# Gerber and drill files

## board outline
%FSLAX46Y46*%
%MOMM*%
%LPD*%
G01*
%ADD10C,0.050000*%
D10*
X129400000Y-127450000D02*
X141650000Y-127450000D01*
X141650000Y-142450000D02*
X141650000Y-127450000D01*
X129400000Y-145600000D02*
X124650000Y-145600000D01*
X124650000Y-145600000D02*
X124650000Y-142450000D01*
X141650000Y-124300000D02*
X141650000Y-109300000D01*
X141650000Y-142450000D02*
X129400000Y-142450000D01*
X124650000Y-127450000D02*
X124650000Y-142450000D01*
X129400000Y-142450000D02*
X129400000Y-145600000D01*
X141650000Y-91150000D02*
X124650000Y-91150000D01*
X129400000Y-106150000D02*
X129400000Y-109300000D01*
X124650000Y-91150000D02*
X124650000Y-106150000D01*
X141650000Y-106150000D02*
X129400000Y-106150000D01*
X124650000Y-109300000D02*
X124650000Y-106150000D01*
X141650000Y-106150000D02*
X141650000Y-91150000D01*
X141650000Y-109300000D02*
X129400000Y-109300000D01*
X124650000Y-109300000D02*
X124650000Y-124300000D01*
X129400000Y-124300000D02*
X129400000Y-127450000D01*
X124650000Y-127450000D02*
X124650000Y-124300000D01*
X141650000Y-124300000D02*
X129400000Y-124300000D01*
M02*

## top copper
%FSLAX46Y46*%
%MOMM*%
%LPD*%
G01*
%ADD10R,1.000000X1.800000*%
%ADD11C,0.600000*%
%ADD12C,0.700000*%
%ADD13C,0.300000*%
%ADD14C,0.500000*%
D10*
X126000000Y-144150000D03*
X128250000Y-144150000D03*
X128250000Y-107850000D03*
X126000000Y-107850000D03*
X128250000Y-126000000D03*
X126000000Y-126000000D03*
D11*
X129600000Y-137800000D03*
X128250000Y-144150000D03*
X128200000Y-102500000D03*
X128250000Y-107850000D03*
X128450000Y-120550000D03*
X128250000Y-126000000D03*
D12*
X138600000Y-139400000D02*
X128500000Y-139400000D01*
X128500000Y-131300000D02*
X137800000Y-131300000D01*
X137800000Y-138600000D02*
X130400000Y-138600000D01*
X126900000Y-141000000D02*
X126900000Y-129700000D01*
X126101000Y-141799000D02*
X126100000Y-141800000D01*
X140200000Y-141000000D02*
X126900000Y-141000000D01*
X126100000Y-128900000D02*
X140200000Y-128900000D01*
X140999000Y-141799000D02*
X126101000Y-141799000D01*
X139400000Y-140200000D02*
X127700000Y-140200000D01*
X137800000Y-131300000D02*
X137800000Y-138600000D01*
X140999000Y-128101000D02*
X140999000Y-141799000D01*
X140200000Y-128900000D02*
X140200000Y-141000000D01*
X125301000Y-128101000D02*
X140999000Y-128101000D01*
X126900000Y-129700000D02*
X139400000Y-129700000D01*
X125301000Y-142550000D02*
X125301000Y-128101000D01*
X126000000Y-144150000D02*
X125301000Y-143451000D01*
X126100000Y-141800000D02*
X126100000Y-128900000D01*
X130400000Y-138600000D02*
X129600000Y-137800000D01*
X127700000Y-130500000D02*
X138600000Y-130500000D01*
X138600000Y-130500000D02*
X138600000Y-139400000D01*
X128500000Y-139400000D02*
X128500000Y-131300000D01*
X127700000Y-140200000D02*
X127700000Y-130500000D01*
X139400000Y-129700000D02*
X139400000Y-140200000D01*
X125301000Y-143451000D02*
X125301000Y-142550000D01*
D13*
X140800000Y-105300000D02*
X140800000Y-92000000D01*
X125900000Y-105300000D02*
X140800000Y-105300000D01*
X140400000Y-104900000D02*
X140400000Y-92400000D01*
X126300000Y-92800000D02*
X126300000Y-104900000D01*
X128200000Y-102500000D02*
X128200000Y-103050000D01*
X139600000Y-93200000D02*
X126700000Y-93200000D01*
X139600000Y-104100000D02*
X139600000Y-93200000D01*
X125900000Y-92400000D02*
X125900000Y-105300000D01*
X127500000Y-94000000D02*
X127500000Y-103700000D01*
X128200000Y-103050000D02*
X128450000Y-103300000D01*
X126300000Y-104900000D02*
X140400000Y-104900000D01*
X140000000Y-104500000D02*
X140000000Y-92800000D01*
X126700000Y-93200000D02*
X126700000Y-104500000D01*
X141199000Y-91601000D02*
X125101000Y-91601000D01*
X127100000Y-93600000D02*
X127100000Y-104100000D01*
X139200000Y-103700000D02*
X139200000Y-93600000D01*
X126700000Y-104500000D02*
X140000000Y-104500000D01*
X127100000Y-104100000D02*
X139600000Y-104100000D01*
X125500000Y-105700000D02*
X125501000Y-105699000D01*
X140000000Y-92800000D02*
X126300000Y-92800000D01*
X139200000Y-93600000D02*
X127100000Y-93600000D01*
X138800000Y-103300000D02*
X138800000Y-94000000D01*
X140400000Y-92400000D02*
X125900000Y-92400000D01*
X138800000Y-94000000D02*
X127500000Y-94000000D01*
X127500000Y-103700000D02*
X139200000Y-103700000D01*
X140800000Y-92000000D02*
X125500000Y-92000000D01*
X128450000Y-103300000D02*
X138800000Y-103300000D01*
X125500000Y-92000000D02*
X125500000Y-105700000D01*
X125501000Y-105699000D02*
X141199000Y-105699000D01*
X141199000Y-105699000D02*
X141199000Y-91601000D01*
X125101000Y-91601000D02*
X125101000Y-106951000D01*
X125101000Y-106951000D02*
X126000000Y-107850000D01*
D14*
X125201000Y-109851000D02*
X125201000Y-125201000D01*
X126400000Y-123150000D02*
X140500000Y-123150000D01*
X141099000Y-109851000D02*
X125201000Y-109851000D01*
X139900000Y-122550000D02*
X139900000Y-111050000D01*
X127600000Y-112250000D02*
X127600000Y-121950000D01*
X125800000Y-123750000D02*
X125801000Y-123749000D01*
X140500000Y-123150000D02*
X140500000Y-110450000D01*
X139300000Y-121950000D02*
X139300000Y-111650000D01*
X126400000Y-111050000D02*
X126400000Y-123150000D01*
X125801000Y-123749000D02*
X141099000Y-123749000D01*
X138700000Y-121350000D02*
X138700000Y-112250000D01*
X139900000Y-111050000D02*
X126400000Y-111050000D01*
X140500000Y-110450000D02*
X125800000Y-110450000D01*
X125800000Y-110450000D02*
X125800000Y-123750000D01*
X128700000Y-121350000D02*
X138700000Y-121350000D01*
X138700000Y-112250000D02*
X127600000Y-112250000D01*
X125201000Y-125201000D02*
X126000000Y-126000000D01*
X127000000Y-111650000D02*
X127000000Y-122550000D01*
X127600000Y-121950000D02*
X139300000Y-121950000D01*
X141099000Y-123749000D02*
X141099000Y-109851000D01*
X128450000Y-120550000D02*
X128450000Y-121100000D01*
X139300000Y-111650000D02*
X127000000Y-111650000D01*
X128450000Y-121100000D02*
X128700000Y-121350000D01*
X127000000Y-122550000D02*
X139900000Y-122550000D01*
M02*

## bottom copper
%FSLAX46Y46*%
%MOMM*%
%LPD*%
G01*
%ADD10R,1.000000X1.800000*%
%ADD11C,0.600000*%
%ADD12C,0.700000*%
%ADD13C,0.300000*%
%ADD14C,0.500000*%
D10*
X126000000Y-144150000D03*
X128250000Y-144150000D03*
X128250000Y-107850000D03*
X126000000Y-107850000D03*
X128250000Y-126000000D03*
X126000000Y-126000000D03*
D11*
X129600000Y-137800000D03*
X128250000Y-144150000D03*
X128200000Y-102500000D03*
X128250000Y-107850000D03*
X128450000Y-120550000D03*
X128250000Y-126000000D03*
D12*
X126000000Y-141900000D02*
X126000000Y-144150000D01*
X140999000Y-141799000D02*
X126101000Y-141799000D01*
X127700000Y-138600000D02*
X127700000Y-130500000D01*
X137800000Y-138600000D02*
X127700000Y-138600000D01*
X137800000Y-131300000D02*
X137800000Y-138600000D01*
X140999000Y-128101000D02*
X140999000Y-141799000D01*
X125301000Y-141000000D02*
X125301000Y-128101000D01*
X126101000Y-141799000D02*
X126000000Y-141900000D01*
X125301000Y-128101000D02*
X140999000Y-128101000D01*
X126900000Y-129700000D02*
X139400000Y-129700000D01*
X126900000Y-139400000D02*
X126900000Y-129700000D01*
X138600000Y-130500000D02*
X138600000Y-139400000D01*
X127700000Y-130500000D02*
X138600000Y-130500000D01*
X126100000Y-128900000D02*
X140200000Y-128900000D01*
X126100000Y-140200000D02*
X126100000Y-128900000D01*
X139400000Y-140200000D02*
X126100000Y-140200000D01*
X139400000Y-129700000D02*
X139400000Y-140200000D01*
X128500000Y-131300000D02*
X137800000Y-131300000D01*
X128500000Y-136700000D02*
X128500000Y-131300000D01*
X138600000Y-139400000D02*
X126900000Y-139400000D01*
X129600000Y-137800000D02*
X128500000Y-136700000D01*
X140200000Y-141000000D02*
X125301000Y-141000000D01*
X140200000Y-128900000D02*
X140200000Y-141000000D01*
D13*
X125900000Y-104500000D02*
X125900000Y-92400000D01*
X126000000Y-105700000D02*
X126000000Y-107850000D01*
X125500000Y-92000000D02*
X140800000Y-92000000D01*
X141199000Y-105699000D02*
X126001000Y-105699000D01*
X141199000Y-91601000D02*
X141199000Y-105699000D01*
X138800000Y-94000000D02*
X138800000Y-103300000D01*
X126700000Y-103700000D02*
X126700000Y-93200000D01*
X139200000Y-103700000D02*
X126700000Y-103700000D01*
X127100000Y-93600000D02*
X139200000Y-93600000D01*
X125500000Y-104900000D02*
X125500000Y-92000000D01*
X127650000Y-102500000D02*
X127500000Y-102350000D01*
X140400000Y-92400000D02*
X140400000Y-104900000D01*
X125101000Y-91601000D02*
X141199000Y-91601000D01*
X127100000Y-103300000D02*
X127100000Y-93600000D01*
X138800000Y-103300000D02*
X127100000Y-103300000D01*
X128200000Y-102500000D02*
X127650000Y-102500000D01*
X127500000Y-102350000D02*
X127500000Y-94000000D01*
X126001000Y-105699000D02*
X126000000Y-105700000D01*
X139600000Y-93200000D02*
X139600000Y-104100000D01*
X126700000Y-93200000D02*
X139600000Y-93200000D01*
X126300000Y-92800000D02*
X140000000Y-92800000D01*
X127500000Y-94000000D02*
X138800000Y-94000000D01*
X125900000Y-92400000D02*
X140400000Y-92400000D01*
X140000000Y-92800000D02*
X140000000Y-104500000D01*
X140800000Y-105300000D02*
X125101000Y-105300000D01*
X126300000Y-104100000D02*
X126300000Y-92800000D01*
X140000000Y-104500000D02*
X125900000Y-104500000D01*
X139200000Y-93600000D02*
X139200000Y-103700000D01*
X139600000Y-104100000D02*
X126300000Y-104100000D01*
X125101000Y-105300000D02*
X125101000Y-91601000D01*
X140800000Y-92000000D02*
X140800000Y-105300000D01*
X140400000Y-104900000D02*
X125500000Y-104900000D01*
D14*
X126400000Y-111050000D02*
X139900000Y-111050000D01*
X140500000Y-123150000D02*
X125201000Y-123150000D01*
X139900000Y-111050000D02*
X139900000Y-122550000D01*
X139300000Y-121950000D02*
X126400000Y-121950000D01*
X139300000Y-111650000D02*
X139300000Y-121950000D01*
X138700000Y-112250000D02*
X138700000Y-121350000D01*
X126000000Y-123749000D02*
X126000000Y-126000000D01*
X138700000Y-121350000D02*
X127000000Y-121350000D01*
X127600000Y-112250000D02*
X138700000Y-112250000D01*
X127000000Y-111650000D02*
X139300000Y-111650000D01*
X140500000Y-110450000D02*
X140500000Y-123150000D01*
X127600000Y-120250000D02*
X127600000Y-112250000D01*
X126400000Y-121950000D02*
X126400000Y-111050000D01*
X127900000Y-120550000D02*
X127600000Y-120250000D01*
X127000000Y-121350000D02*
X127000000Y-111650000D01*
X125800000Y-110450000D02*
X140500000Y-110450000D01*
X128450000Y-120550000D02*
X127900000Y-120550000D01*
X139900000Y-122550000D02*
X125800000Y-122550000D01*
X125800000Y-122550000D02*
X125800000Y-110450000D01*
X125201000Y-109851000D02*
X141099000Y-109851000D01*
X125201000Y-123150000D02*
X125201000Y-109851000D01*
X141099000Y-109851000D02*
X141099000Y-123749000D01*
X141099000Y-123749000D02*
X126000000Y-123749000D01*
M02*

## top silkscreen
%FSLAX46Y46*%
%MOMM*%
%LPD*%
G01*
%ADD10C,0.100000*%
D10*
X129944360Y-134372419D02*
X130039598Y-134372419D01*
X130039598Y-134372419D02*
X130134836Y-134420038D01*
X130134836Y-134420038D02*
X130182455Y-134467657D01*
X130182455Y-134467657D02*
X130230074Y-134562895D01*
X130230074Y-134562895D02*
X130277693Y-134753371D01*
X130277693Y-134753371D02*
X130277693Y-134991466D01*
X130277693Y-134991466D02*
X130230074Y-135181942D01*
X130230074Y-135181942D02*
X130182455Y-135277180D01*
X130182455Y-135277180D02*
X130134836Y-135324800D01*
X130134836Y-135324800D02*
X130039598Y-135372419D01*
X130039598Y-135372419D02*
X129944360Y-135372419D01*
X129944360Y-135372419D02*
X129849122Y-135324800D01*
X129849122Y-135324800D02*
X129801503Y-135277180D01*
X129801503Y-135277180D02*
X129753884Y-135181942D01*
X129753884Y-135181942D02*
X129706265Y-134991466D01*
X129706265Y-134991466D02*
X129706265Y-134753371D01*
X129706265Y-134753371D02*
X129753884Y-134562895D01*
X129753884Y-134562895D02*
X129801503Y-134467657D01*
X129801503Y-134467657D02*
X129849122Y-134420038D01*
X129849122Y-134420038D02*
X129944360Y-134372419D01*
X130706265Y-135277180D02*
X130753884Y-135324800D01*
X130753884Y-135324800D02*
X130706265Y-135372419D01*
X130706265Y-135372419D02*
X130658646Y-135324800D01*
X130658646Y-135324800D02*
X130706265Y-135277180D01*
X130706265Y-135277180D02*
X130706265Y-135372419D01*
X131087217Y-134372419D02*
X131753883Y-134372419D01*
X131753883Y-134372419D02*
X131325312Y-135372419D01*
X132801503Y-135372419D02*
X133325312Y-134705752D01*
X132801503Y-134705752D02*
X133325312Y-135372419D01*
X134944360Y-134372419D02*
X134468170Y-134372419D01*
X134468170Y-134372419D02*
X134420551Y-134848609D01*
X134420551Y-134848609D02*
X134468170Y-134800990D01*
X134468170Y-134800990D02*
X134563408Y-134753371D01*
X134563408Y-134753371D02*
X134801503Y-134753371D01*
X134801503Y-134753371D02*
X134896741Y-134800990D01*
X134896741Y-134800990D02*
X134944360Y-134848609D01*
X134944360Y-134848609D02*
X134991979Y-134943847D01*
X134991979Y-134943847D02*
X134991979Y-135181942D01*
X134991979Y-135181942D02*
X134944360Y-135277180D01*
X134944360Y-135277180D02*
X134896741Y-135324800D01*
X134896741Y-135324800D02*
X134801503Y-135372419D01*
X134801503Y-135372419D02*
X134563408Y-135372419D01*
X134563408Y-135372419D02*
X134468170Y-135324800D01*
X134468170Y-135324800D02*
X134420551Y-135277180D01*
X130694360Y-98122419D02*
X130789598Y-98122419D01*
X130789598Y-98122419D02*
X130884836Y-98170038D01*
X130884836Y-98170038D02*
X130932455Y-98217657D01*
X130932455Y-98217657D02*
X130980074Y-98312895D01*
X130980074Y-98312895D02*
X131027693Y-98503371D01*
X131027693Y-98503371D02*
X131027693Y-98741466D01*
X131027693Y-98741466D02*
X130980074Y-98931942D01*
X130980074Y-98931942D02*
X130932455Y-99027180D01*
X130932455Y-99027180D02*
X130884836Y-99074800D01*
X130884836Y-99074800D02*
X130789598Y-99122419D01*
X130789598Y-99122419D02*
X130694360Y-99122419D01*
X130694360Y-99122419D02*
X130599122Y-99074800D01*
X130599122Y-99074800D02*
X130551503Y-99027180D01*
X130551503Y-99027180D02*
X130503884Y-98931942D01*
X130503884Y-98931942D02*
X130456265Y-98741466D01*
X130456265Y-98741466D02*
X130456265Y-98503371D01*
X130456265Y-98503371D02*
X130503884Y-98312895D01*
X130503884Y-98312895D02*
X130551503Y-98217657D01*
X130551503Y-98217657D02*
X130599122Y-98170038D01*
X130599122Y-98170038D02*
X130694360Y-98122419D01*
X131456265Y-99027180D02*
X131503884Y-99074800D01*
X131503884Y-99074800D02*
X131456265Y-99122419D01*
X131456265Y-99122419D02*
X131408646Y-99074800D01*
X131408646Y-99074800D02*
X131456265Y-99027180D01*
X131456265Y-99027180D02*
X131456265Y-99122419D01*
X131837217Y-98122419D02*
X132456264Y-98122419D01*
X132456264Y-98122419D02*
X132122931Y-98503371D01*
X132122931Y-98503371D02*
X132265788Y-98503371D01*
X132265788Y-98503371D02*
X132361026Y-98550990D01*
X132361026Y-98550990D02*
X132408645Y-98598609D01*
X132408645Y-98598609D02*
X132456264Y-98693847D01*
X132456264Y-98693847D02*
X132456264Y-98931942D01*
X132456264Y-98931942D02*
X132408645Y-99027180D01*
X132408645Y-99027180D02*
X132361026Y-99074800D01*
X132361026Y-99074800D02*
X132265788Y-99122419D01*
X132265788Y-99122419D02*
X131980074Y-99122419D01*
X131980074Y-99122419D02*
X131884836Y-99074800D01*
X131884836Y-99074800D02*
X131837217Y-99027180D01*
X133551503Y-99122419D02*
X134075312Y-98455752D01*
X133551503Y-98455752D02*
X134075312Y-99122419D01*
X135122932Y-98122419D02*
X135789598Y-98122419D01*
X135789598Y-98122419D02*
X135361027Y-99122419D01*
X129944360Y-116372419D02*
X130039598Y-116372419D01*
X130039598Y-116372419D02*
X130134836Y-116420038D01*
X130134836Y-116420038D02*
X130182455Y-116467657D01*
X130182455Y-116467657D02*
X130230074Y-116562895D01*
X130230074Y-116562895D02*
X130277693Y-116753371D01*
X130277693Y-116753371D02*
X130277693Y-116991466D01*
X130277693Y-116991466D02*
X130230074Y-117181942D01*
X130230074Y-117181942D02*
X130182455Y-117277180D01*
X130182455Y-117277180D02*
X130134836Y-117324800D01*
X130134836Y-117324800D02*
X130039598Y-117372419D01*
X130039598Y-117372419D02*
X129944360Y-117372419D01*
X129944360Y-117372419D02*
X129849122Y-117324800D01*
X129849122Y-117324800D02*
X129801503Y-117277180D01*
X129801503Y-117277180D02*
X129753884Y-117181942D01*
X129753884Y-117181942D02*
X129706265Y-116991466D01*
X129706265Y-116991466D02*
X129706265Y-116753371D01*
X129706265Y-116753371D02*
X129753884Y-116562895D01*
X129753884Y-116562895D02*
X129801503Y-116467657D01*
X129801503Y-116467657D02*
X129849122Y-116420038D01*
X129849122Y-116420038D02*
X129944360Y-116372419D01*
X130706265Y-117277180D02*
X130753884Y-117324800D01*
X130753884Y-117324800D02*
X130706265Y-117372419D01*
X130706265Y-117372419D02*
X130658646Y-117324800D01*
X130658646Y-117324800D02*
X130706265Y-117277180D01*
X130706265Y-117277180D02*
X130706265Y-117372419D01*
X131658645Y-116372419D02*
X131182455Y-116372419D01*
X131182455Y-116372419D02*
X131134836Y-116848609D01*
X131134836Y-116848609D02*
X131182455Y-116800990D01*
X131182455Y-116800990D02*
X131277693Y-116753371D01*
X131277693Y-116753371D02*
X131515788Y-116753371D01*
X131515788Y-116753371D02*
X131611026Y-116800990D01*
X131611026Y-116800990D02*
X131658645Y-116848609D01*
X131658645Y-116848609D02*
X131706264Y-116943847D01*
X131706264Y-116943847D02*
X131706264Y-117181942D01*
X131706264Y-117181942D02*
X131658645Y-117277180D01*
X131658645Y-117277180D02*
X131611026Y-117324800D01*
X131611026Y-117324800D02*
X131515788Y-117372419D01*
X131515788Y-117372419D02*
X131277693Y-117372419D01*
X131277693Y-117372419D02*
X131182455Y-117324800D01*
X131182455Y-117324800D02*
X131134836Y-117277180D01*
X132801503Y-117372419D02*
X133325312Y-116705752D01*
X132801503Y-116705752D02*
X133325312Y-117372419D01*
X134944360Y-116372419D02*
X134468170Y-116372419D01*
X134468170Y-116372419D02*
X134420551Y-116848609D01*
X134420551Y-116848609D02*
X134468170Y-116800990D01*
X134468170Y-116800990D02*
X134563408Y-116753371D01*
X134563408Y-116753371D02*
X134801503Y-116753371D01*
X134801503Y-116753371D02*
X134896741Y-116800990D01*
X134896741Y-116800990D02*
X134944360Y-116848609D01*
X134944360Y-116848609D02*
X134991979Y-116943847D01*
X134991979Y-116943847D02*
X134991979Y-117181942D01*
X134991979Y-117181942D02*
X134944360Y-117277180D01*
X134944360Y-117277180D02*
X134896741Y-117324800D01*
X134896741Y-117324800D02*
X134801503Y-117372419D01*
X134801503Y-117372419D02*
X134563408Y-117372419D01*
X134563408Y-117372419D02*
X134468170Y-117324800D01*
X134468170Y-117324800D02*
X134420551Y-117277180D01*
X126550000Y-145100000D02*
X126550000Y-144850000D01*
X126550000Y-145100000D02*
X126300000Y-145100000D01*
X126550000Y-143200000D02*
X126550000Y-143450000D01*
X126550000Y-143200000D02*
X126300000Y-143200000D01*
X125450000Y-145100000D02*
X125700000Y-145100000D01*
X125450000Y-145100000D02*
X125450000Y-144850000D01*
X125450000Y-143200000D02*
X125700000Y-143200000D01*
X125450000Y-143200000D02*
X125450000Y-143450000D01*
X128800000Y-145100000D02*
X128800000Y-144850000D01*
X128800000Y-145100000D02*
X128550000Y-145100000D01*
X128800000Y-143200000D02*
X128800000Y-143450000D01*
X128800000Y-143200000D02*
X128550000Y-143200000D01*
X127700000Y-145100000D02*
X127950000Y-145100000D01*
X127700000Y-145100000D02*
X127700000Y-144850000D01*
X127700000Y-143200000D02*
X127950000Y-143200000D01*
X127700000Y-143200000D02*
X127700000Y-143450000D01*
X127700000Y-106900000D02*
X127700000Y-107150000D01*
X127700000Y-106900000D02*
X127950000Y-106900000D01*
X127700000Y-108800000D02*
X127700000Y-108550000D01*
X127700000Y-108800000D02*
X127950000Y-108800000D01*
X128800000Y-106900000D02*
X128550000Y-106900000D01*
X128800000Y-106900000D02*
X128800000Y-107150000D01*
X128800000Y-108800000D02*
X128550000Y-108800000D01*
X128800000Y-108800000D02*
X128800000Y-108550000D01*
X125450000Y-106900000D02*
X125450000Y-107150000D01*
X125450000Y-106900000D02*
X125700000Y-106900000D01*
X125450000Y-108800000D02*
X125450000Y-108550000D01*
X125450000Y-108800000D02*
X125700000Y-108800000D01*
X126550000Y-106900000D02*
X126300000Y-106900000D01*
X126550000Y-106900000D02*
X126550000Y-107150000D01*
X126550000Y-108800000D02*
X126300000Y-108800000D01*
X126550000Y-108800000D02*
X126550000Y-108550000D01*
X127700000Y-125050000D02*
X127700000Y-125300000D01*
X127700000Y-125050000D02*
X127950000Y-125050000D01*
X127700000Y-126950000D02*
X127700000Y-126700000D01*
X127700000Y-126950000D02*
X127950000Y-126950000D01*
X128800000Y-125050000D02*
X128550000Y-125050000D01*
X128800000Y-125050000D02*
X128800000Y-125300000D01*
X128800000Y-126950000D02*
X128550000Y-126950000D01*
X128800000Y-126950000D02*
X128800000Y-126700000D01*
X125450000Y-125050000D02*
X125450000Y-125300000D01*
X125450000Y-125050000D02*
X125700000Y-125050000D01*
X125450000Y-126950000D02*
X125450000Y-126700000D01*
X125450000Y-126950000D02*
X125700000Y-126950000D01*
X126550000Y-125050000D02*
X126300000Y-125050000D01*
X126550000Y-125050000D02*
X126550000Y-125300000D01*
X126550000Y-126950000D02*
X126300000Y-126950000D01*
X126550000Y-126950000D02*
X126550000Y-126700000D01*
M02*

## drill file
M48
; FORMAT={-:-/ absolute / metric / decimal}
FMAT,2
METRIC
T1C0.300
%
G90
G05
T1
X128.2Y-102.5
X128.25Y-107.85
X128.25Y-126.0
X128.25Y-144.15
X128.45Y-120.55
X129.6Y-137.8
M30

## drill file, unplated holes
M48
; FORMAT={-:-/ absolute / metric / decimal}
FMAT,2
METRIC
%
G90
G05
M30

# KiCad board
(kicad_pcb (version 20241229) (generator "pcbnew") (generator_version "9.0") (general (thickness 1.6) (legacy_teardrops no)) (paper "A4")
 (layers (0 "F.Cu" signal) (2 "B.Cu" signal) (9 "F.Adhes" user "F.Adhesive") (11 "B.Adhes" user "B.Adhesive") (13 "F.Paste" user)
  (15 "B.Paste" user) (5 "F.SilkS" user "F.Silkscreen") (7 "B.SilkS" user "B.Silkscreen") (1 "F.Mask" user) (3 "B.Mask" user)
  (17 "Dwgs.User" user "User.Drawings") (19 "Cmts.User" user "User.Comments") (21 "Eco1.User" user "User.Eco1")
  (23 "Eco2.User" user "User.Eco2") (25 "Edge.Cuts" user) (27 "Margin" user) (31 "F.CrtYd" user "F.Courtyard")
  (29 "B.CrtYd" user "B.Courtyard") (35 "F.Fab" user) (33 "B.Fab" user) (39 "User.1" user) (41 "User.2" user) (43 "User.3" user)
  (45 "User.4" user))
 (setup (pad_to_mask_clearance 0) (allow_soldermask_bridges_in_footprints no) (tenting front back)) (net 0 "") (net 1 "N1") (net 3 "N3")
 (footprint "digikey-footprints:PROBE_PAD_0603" (layer "F.Cu") (at 128.25 126 90)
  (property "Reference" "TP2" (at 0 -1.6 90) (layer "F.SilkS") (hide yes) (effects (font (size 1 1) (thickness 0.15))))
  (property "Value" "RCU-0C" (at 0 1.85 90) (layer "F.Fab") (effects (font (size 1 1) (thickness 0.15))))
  (fp_line (start 0.95 -0.55) (end 0.7 -0.55) (stroke (width 0.1) (type solid)) (layer "F.SilkS"))
  (fp_line (start 0.95 -0.55) (end 0.95 -0.3) (stroke (width 0.1) (type solid)) (layer "F.SilkS"))
  (fp_line (start -0.95 -0.55) (end -0.7 -0.55) (stroke (width 0.1) (type solid)) (layer "F.SilkS"))
  (fp_line (start -0.95 -0.55) (end -0.95 -0.3) (stroke (width 0.1) (type solid)) (layer "F.SilkS"))
  (fp_line (start 0.95 0.55) (end 0.95 0.3) (stroke (width 0.1) (type solid)) (layer "F.SilkS"))
  (fp_line (start 0.95 0.55) (end 0.7 0.55) (stroke (width 0.1) (type solid)) (layer "F.SilkS"))
  (fp_line (start -0.95 0.55) (end -0.95 0.3) (stroke (width 0.1) (type solid)) (layer "F.SilkS"))
  (fp_line (start -0.95 0.55) (end -0.7 0.55) (stroke (width 0.1) (type solid)) (layer "F.SilkS"))
  (pad "1" smd rect (at 0 0 90) (size 1.8 1) (layers "F.Cu" "F.Mask" "F.Paste") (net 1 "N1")))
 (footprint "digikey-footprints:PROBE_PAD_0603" (layer "F.Cu") (at 126 107.85 90)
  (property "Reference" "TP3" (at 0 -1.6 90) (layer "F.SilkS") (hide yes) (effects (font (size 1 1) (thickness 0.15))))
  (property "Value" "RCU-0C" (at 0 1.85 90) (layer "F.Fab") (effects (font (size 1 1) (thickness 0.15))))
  (fp_line (start 0.95 -0.55) (end 0.7 -0.55) (stroke (width 0.1) (type solid)) (layer "F.SilkS") (net 2))
  (fp_line (start 0.95 -0.55) (end 0.95 -0.3) (stroke (width 0.1) (type solid)) (layer "F.SilkS") (net 2))
  (fp_line (start -0.95 -0.55) (end -0.7 -0.55) (stroke (width 0.1) (type solid)) (layer "F.SilkS") (net 2))
  (fp_line (start -0.95 -0.55) (end -0.95 -0.3) (stroke (width 0.1) (type solid)) (layer "F.SilkS") (net 2))
  (fp_line (start 0.95 0.55) (end 0.95 0.3) (stroke (width 0.1) (type solid)) (layer "F.SilkS") (net 2))
  (fp_line (start 0.95 0.55) (end 0.7 0.55) (stroke (width 0.1) (type solid)) (layer "F.SilkS") (net 2))
  (fp_line (start -0.95 0.55) (end -0.95 0.3) (stroke (width 0.1) (type solid)) (layer "F.SilkS") (net 2))
  (fp_line (start -0.95 0.55) (end -0.7 0.55) (stroke (width 0.1) (type solid)) (layer "F.SilkS") (net 2))
  (pad "1" smd rect (at 0 0 90) (size 1.8 1) (layers "F.Cu" "F.Mask" "F.Paste") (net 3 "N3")))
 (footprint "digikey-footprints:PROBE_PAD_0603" (layer "F.Cu") (at 126 126 90)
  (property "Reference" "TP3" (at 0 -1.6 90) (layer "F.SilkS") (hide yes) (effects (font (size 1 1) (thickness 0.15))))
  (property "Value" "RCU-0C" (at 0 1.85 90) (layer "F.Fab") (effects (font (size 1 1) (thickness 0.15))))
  (fp_line (start 0.95 -0.55) (end 0.7 -0.55) (stroke (width 0.1) (type solid)) (layer "F.SilkS"))
  (fp_line (start 0.95 -0.55) (end 0.95 -0.3) (stroke (width 0.1) (type solid)) (layer "F.SilkS"))
  (fp_line (start -0.95 -0.55) (end -0.7 -0.55) (stroke (width 0.1) (type solid)) (layer "F.SilkS"))
  (fp_line (start -0.95 -0.55) (end -0.95 -0.3) (stroke (width 0.1) (type solid)) (layer "F.SilkS"))
  (fp_line (start 0.95 0.55) (end 0.95 0.3) (stroke (width 0.1) (type solid)) (layer "F.SilkS"))
  (fp_line (start 0.95 0.55) (end 0.7 0.55) (stroke (width 0.1) (type solid)) (layer "F.SilkS"))
  (fp_line (start -0.95 0.55) (end -0.95 0.3) (stroke (width 0.1) (type solid)) (layer "F.SilkS"))
  (fp_line (start -0.95 0.55) (end -0.7 0.55) (stroke (width 0.1) (type solid)) (layer "F.SilkS"))
  (pad "1" smd rect (at 0 0 90) (size 1.8 1) (layers "F.Cu" "F.Mask" "F.Paste") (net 3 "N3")))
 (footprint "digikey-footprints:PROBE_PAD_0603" (layer "F.Cu") (at 128.25 144.15 90)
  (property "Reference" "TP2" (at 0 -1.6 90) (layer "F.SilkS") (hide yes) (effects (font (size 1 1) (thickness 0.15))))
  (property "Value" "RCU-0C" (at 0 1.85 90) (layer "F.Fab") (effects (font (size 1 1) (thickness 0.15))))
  (fp_line (start 0.95 -0.55) (end 0.7 -0.55) (stroke (width 0.1) (type solid)) (layer "F.SilkS") (net 4))
  (fp_line (start 0.95 -0.55) (end 0.95 -0.3) (stroke (width 0.1) (type solid)) (layer "F.SilkS") (net 4))
  (fp_line (start -0.95 -0.55) (end -0.7 -0.55) (stroke (width 0.1) (type solid)) (layer "F.SilkS") (net 4))
  (fp_line (start -0.95 -0.55) (end -0.95 -0.3) (stroke (width 0.1) (type solid)) (layer "F.SilkS") (net 4))
  (fp_line (start 0.95 0.55) (end 0.95 0.3) (stroke (width 0.1) (type solid)) (layer "F.SilkS") (net 4))
  (fp_line (start 0.95 0.55) (end 0.7 0.55) (stroke (width 0.1) (type solid)) (layer "F.SilkS") (net 4))
  (fp_line (start -0.95 0.55) (end -0.95 0.3) (stroke (width 0.1) (type solid)) (layer "F.SilkS") (net 4))
  (fp_line (start -0.95 0.55) (end -0.7 0.55) (stroke (width 0.1) (type solid)) (layer "F.SilkS") (net 4))
  (pad "1" smd rect (at 0 0 90) (size 1.8 1) (layers "F.Cu" "F.Mask" "F.Paste") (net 1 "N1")))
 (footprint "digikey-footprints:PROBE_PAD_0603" (layer "F.Cu") (at 126 144.15 90)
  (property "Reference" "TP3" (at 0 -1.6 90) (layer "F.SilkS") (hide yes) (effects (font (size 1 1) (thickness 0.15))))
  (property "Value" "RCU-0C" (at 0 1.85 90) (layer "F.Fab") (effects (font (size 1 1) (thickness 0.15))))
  (fp_line (start 0.95 -0.55) (end 0.7 -0.55) (stroke (width 0.1) (type solid)) (layer "F.SilkS") (net 4))
  (fp_line (start 0.95 -0.55) (end 0.95 -0.3) (stroke (width 0.1) (type solid)) (layer "F.SilkS") (net 4))
  (fp_line (start -0.95 -0.55) (end -0.7 -0.55) (stroke (width 0.1) (type solid)) (layer "F.SilkS") (net 4))
  (fp_line (start -0.95 -0.55) (end -0.95 -0.3) (stroke (width 0.1) (type solid)) (layer "F.SilkS") (net 4))
  (fp_line (start 0.95 0.55) (end 0.95 0.3) (stroke (width 0.1) (type solid)) (layer "F.SilkS") (net 4))
  (fp_line (start 0.95 0.55) (end 0.7 0.55) (stroke (width 0.1) (type solid)) (layer "F.SilkS") (net 4))
  (fp_line (start -0.95 0.55) (end -0.95 0.3) (stroke (width 0.1) (type solid)) (layer "F.SilkS") (net 4))
  (fp_line (start -0.95 0.55) (end -0.7 0.55) (stroke (width 0.1) (type solid)) (layer "F.SilkS") (net 4))
  (pad "1" smd rect (at 0 0 90) (size 1.8 1) (layers "F.Cu" "F.Mask" "F.Paste") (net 3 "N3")))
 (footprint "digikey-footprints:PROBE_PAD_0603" (layer "F.Cu") (at 128.25 107.85 90)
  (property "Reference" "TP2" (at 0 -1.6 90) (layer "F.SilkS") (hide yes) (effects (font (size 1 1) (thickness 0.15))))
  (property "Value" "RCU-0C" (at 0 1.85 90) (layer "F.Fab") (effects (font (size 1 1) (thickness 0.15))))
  (fp_line (start 0.95 -0.55) (end 0.7 -0.55) (stroke (width 0.1) (type solid)) (layer "F.SilkS") (net 2))
  (fp_line (start 0.95 -0.55) (end 0.95 -0.3) (stroke (width 0.1) (type solid)) (layer "F.SilkS") (net 2))
  (fp_line (start -0.95 -0.55) (end -0.7 -0.55) (stroke (width 0.1) (type solid)) (layer "F.SilkS") (net 2))
  (fp_line (start -0.95 -0.55) (end -0.95 -0.3) (stroke (width 0.1) (type solid)) (layer "F.SilkS") (net 2))
  (fp_line (start 0.95 0.55) (end 0.95 0.3) (stroke (width 0.1) (type solid)) (layer "F.SilkS") (net 2))
  (fp_line (start 0.95 0.55) (end 0.7 0.55) (stroke (width 0.1) (type solid)) (layer "F.SilkS") (net 2))
  (fp_line (start -0.95 0.55) (end -0.95 0.3) (stroke (width 0.1) (type solid)) (layer "F.SilkS") (net 2))
  (fp_line (start -0.95 0.55) (end -0.7 0.55) (stroke (width 0.1) (type solid)) (layer "F.SilkS") (net 2))
  (pad "1" smd rect (at 0 0 90) (size 1.8 1) (layers "F.Cu" "F.Mask" "F.Paste") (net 1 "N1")))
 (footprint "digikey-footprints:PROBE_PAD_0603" (layer "B.Cu") (at 128.25 144.15 90)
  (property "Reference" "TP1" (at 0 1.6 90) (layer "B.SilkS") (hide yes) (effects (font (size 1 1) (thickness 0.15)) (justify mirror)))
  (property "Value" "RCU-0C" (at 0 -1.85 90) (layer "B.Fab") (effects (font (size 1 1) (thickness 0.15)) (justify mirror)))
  (pad "1" smd rect (at 0 0 90) (size 1.8 1) (layers "B.Cu" "B.Mask" "B.Paste") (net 1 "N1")))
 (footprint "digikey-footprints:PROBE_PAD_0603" (layer "B.Cu") (at 126 144.15 90)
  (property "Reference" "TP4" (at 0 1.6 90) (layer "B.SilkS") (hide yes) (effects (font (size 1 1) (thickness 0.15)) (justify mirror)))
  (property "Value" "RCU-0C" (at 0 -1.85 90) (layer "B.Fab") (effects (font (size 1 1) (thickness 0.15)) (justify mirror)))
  (pad "1" smd rect (at 0 0 90) (size 1.8 1) (layers "B.Cu" "B.Mask" "B.Paste") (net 3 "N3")))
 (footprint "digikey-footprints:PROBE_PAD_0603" (layer "B.Cu") (at 126 107.85 90)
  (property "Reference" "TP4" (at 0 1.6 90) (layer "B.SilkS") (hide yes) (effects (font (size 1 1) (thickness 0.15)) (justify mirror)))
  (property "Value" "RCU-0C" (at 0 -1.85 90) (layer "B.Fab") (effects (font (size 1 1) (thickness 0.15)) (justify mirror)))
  (pad "1" smd rect (at 0 0 90) (size 1.8 1) (layers "B.Cu" "B.Mask" "B.Paste") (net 3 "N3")))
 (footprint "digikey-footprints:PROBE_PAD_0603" (layer "B.Cu") (at 128.25 126 90)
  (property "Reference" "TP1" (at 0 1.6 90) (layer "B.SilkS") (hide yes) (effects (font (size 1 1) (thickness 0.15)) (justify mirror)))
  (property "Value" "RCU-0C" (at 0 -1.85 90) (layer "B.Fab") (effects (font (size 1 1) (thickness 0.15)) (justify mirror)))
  (pad "1" smd rect (at 0 0 90) (size 1.8 1) (layers "B.Cu" "B.Mask" "B.Paste") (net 1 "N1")))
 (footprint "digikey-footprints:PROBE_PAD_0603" (layer "B.Cu") (at 128.25 107.85 90)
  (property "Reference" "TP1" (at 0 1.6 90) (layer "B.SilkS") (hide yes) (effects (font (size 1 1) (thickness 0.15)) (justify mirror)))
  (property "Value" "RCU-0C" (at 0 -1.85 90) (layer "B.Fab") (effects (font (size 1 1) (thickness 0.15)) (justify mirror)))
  (pad "1" smd rect (at 0 0 90) (size 1.8 1) (layers "B.Cu" "B.Mask" "B.Paste") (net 1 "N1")))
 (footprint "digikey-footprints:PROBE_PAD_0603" (layer "B.Cu") (at 126 126 90)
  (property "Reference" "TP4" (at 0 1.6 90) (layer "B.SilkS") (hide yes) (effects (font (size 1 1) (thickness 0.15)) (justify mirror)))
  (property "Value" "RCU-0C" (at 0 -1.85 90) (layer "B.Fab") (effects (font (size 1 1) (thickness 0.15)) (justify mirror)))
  (pad "1" smd rect (at 0 0 90) (size 1.8 1) (layers "B.Cu" "B.Mask" "B.Paste") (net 3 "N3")))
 (gr_line (start 141.65 109.3) (end 129.4 109.3) (stroke (width 0.05) (type default)) (layer "Edge.Cuts"))
 (gr_line (start 141.65 142.45) (end 129.4 142.45) (stroke (width 0.05) (type default)) (layer "Edge.Cuts"))
 (gr_line (start 141.65 106.15) (end 141.65 91.15) (stroke (width 0.05) (type default)) (layer "Edge.Cuts"))
 (gr_line (start 141.65 91.15) (end 124.65 91.15) (stroke (width 0.05) (type default)) (layer "Edge.Cuts"))
 (gr_line (start 124.65 91.15) (end 124.65 106.15) (stroke (width 0.05) (type default)) (layer "Edge.Cuts"))
 (gr_line (start 129.4 127.45) (end 141.65 127.45) (stroke (width 0.05) (type default)) (layer "Edge.Cuts"))
 (gr_line (start 129.4 145.6) (end 124.65 145.6) (stroke (width 0.05) (type default)) (layer "Edge.Cuts"))
 (gr_line (start 141.65 142.45) (end 141.65 127.45) (stroke (width 0.05) (type default)) (layer "Edge.Cuts"))
 (gr_line (start 124.65 127.45) (end 124.65 142.45) (stroke (width 0.05) (type default)) (layer "Edge.Cuts"))
 (gr_line (start 124.65 145.6) (end 124.65 142.45) (stroke (width 0.05) (type default)) (layer "Edge.Cuts"))
 (gr_line (start 129.4 106.15) (end 129.4 109.3) (stroke (width 0.05) (type default)) (layer "Edge.Cuts"))
 (gr_line (start 141.65 106.15) (end 129.4 106.15) (stroke (width 0.05) (type default)) (layer "Edge.Cuts"))
 (gr_line (start 141.65 124.3) (end 141.65 109.3) (stroke (width 0.05) (type default)) (layer "Edge.Cuts"))
 (gr_line (start 124.65 109.3) (end 124.65 124.3) (stroke (width 0.05) (type default)) (layer "Edge.Cuts"))
 (gr_line (start 129.4 124.3) (end 129.4 127.45) (stroke (width 0.05) (type default)) (layer "Edge.Cuts"))
 (gr_line (start 124.65 127.45) (end 124.65 124.3) (stroke (width 0.05) (type default)) (layer "Edge.Cuts"))
 (gr_line (start 141.65 124.3) (end 129.4 124.3) (stroke (width 0.05) (type default)) (layer "Edge.Cuts"))
 (gr_line (start 129.4 142.45) (end 129.4 145.6) (stroke (width 0.05) (type default)) (layer "Edge.Cuts"))
 (gr_line (start 124.65 109.3) (end 124.65 106.15) (stroke (width 0.05) (type default)) (layer "Edge.Cuts"))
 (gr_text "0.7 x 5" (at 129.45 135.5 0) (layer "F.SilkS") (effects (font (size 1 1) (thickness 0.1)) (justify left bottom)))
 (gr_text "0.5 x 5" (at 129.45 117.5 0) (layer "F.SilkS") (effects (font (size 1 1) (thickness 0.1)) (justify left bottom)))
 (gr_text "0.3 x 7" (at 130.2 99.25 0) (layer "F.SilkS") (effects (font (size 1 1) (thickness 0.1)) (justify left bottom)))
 (via (at 128.25 144.15) (size 0.6) (drill 0.3) (layers "F.Cu" "B.Cu") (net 1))
 (via (at 128.25 107.85) (size 0.6) (drill 0.3) (layers "F.Cu" "B.Cu") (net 1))
 (via (at 128.25 126) (size 0.6) (drill 0.3) (layers "F.Cu" "B.Cu") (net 1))
 (segment (start 126.1 141.8) (end 126.1 128.9) (width 0.7) (layer "F.Cu") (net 3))
 (segment (start 125.301 142.55) (end 125.301 128.101) (width 0.7) (layer "F.Cu") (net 3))
 (segment (start 127.5 103.7) (end 139.2 103.7) (width 0.3) (layer "F.Cu") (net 3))
 (segment (start 125.101 106.951) (end 126 107.85) (width 0.3) (layer "F.Cu") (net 3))
 (segment (start 125.201 109.851) (end 125.201 125.201) (width 0.5) (layer "F.Cu") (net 3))
 (segment (start 128.45 120.55) (end 128.45 121.1) (width 0.5) (layer "F.Cu") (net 3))
 (segment (start 127 122.55) (end 139.9 122.55) (width 0.5) (layer "F.Cu") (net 3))
 (segment (start 127 111.65) (end 127 122.55) (width 0.5) (layer "F.Cu") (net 3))
 (segment (start 128.45 121.1) (end 128.7 121.35) (width 0.5) (layer "F.Cu") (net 3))
 (segment (start 138.7 121.35) (end 138.7 112.25) (width 0.5) (layer "F.Cu") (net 3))
 (segment (start 125.9 92.4) (end 125.9 105.3) (width 0.3) (layer "F.Cu") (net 3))
 (segment (start 140 104.5) (end 140 92.8) (width 0.3) (layer "F.Cu") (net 3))
 (segment (start 126.3 104.9) (end 140.4 104.9) (width 0.3) (layer "F.Cu") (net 3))
 (segment (start 139.6 93.2) (end 126.7 93.2) (width 0.3) (layer "F.Cu") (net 3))
 (segment (start 141.099 123.749) (end 141.099 109.851) (width 0.5) (layer "F.Cu") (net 3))
 (segment (start 139.9 122.55) (end 139.9 111.05) (width 0.5) (layer "F.Cu") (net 3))
 (segment (start 126.1 128.9) (end 140.2 128.9) (width 0.7) (layer "F.Cu") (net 3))
 (segment (start 127.1 93.6) (end 127.1 104.1) (width 0.3) (layer "F.Cu") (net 3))
 (segment (start 125.201 125.201) (end 126 126) (width 0.5) (layer "F.Cu") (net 3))
 (segment (start 126.9 141) (end 126.9 129.7) (width 0.7) (layer "F.Cu") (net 3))
 (segment (start 139.2 103.7) (end 139.2 93.6) (width 0.3) (layer "F.Cu") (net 3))
 (segment (start 140.999 128.101) (end 140.999 141.799) (width 0.7) (layer "F.Cu") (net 3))
 (segment (start 128.45 103.3) (end 138.8 103.3) (width 0.3) (layer "F.Cu") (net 3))
 (segment (start 137.8 138.6) (end 130.4 138.6) (width 0.7) (layer "F.Cu") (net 3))
 (segment (start 140.2 141) (end 126.9 141) (width 0.7) (layer "F.Cu") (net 3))
 (segment (start 127.5 94) (end 127.5 103.7) (width 0.3) (layer "F.Cu") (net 3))
 (segment (start 138.6 139.4) (end 128.5 139.4) (width 0.7) (layer "F.Cu") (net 3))
 (segment (start 125.301 143.451) (end 125.301 142.55) (width 0.7) (layer "F.Cu") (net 3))
 (segment (start 127.7 140.2) (end 127.7 130.5) (width 0.7) (layer "F.Cu") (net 3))
 (segment (start 139.3 121.95) (end 139.3 111.65) (width 0.5) (layer "F.Cu") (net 3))
 (segment (start 140.5 123.15) (end 140.5 110.45) (width 0.5) (layer "F.Cu") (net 3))
 (segment (start 139.6 104.1) (end 139.6 93.2) (width 0.3) (layer "F.Cu") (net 3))
 (segment (start 139.2 93.6) (end 127.1 93.6) (width 0.3) (layer "F.Cu") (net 3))
 (segment (start 125.101 91.601) (end 125.101 106.951) (width 0.3) (layer "F.Cu") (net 3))
 (segment (start 141.099 109.851) (end 125.201 109.851) (width 0.5) (layer "F.Cu") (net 3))
 (segment (start 125.501 105.699) (end 141.199 105.699) (width 0.3) (layer "F.Cu") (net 3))
 (segment (start 137.8 131.3) (end 137.8 138.6) (width 0.7) (layer "F.Cu") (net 3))
 (segment (start 139.4 140.2) (end 127.7 140.2) (width 0.7) (layer "F.Cu") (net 3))
 (segment (start 125.9 105.3) (end 140.8 105.3) (width 0.3) (layer "F.Cu") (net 3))
 (segment (start 128.7 121.35) (end 138.7 121.35) (width 0.5) (layer "F.Cu") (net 3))
 (segment (start 126.101 141.799) (end 126.1 141.8) (width 0.7) (layer "F.Cu") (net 3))
 (segment (start 125.801 123.749) (end 141.099 123.749) (width 0.5) (layer "F.Cu") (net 3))
 (segment (start 126.7 93.2) (end 126.7 104.5) (width 0.3) (layer "F.Cu") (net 3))
 (segment (start 139.4 129.7) (end 139.4 140.2) (width 0.7) (layer "F.Cu") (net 3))
 (segment (start 126.7 104.5) (end 140 104.5) (width 0.3) (layer "F.Cu") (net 3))
 (segment (start 128.5 131.3) (end 137.8 131.3) (width 0.7) (layer "F.Cu") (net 3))
 (segment (start 125.5 92) (end 125.5 105.7) (width 0.3) (layer "F.Cu") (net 3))
 (segment (start 128.2 102.5) (end 128.2 103.05) (width 0.3) (layer "F.Cu") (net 3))
 (segment (start 138.8 94) (end 127.5 94) (width 0.3) (layer "F.Cu") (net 3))
 (segment (start 141.199 105.699) (end 141.199 91.601) (width 0.3) (layer "F.Cu") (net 3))
 (segment (start 127.1 104.1) (end 139.6 104.1) (width 0.3) (layer "F.Cu") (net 3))
 (segment (start 138.7 112.25) (end 127.6 112.25) (width 0.5) (layer "F.Cu") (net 3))
 (segment (start 126.9 129.7) (end 139.4 129.7) (width 0.7) (layer "F.Cu") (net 3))
 (segment (start 140.2 128.9) (end 140.2 141) (width 0.7) (layer "F.Cu") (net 3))
 (segment (start 126.4 123.15) (end 140.5 123.15) (width 0.5) (layer "F.Cu") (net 3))
 (segment (start 140.5 110.45) (end 125.8 110.45) (width 0.5) (layer "F.Cu") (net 3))
 (segment (start 140.8 105.3) (end 140.8 92) (width 0.3) (layer "F.Cu") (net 3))
 (segment (start 126.3 92.8) (end 126.3 104.9) (width 0.3) (layer "F.Cu") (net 3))
 (segment (start 140.999 141.799) (end 126.101 141.799) (width 0.7) (layer "F.Cu") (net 3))
 (segment (start 126 144.15) (end 125.301 143.451) (width 0.7) (layer "F.Cu") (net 3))
 (segment (start 126.4 111.05) (end 126.4 123.15) (width 0.5) (layer "F.Cu") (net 3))
 (segment (start 139.9 111.05) (end 126.4 111.05) (width 0.5) (layer "F.Cu") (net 3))
 (segment (start 127.6 121.95) (end 139.3 121.95) (width 0.5) (layer "F.Cu") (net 3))
 (segment (start 128.5 139.4) (end 128.5 131.3) (width 0.7) (layer "F.Cu") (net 3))
 (segment (start 138.8 103.3) (end 138.8 94) (width 0.3) (layer "F.Cu") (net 3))
 (segment (start 130.4 138.6) (end 129.6 137.8) (width 0.7) (layer "F.Cu") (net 3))
 (segment (start 140.4 92.4) (end 125.9 92.4) (width 0.3) (layer "F.Cu") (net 3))
 (segment (start 125.8 110.45) (end 125.8 123.75) (width 0.5) (layer "F.Cu") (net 3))
 (segment (start 127.6 112.25) (end 127.6 121.95) (width 0.5) (layer "F.Cu") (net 3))
 (segment (start 125.301 128.101) (end 140.999 128.101) (width 0.7) (layer "F.Cu") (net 3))
 (segment (start 140.4 104.9) (end 140.4 92.4) (width 0.3) (layer "F.Cu") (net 3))
 (segment (start 139.3 111.65) (end 127 111.65) (width 0.5) (layer "F.Cu") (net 3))
 (segment (start 141.199 91.601) (end 125.101 91.601) (width 0.3) (layer "F.Cu") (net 3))
 (segment (start 125.5 105.7) (end 125.501 105.699) (width 0.3) (layer "F.Cu") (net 3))
 (segment (start 125.8 123.75) (end 125.801 123.749) (width 0.5) (layer "F.Cu") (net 3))
 (segment (start 128.2 103.05) (end 128.45 103.3) (width 0.3) (layer "F.Cu") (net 3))
 (segment (start 138.6 130.5) (end 138.6 139.4) (width 0.7) (layer "F.Cu") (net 3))
 (segment (start 127.7 130.5) (end 138.6 130.5) (width 0.7) (layer "F.Cu") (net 3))
 (segment (start 140 92.8) (end 126.3 92.8) (width 0.3) (layer "F.Cu") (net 3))
 (segment (start 140.8 92) (end 125.5 92) (width 0.3) (layer "F.Cu") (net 3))
 (via (at 129.6 137.8) (size 0.6) (drill 0.3) (layers "F.Cu" "B.Cu") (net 3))
 (via (at 128.45 120.55) (size 0.6) (drill 0.3) (layers "F.Cu" "B.Cu") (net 3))
 (via (at 128.2 102.5) (size 0.6) (drill 0.3) (layers "F.Cu" "B.Cu") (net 3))
 (segment (start 126.3 104.1) (end 126.3 92.8) (width 0.3) (layer "B.Cu") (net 3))
 (segment (start 141.099 123.749) (end 126 123.749) (width 0.5) (layer "B.Cu") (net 3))
 (segment (start 125.5 92) (end 140.8 92) (width 0.3) (layer "B.Cu") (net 3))
 (segment (start 140.8 92) (end 140.8 105.3) (width 0.3) (layer "B.Cu") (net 3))
 (segment (start 125.201 123.15) (end 125.201 109.851) (width 0.5) (layer "B.Cu") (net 3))
 (segment (start 125.201 109.851) (end 141.099 109.851) (width 0.5) (layer "B.Cu") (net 3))
 (segment (start 127.5 94) (end 138.8 94) (width 0.3) (layer "B.Cu") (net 3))
 (segment (start 139.9 122.55) (end 125.8 122.55) (width 0.5) (layer "B.Cu") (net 3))
 (segment (start 127.6 120.25) (end 127.6 112.25) (width 0.5) (layer "B.Cu") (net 3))
 (segment (start 125.9 104.5) (end 125.9 92.4) (width 0.3) (layer "B.Cu") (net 3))
 (segment (start 127.6 112.25) (end 138.7 112.25) (width 0.5) (layer "B.Cu") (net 3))
 (segment (start 139.6 104.1) (end 126.3 104.1) (width 0.3) (layer "B.Cu") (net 3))
 (segment (start 140.5 110.45) (end 140.5 123.15) (width 0.5) (layer "B.Cu") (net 3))
 (segment (start 139.4 129.7) (end 139.4 140.2) (width 0.7) (layer "B.Cu") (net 3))
 (segment (start 127.5 102.35) (end 127.5 94) (width 0.3) (layer "B.Cu") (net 3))
 (segment (start 139.6 93.2) (end 139.6 104.1) (width 0.3) (layer "B.Cu") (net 3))
 (segment (start 126.101 141.799) (end 126 141.9) (width 0.7) (layer "B.Cu") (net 3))
 (segment (start 140.999 141.799) (end 126.101 141.799) (width 0.7) (layer "B.Cu") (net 3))
 (segment (start 126.1 128.9) (end 140.2 128.9) (width 0.7) (layer "B.Cu") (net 3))
 (segment (start 126.9 139.4) (end 126.9 129.7) (width 0.7) (layer "B.Cu") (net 3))
 (segment (start 138.8 94) (end 138.8 103.3) (width 0.3) (layer "B.Cu") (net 3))
 (segment (start 126.1 140.2) (end 126.1 128.9) (width 0.7) (layer "B.Cu") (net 3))
 (segment (start 125.8 122.55) (end 125.8 110.45) (width 0.5) (layer "B.Cu") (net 3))
 (segment (start 127.9 120.55) (end 127.6 120.25) (width 0.5) (layer "B.Cu") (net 3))
 (segment (start 140.4 104.9) (end 125.5 104.9) (width 0.3) (layer "B.Cu") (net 3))
 (segment (start 127.1 103.3) (end 127.1 93.6) (width 0.3) (layer "B.Cu") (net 3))
 (segment (start 139.9 111.05) (end 139.9 122.55) (width 0.5) (layer "B.Cu") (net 3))
 (segment (start 128.5 136.7) (end 128.5 131.3) (width 0.7) (layer "B.Cu") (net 3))
 (segment (start 126.4 121.95) (end 126.4 111.05) (width 0.5) (layer "B.Cu") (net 3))
 (segment (start 125.301 128.101) (end 140.999 128.101) (width 0.7) (layer "B.Cu") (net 3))
 (segment (start 125.8 110.45) (end 140.5 110.45) (width 0.5) (layer "B.Cu") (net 3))
 (segment (start 128.45 120.55) (end 127.9 120.55) (width 0.5) (layer "B.Cu") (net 3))
 (segment (start 129.6 137.8) (end 128.5 136.7) (width 0.7) (layer "B.Cu") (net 3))
 (segment (start 127 121.35) (end 127 111.65) (width 0.5) (layer "B.Cu") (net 3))
 (segment (start 125.101 105.3) (end 125.101 91.601) (width 0.3) (layer "B.Cu") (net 3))
 (segment (start 140 92.8) (end 140 104.5) (width 0.3) (layer "B.Cu") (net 3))
 (segment (start 127 111.65) (end 139.3 111.65) (width 0.5) (layer "B.Cu") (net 3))
 (segment (start 139.3 111.65) (end 139.3 121.95) (width 0.5) (layer "B.Cu") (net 3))
 (segment (start 125.9 92.4) (end 140.4 92.4) (width 0.3) (layer "B.Cu") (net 3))
 (segment (start 127.1 93.6) (end 139.2 93.6) (width 0.3) (layer "B.Cu") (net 3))
 (segment (start 126 123.749) (end 126 126) (width 0.5) (layer "B.Cu") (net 3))
 (segment (start 126.7 103.7) (end 126.7 93.2) (width 0.3) (layer "B.Cu") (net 3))
 (segment (start 126.7 93.2) (end 139.6 93.2) (width 0.3) (layer "B.Cu") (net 3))
 (segment (start 126.3 92.8) (end 140 92.8) (width 0.3) (layer "B.Cu") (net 3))
 (segment (start 128.2 102.5) (end 127.65 102.5) (width 0.3) (layer "B.Cu") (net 3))
 (segment (start 126 105.7) (end 126 107.85) (width 0.3) (layer "B.Cu") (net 3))
 (segment (start 128.5 131.3) (end 137.8 131.3) (width 0.7) (layer "B.Cu") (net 3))
 (segment (start 140.5 123.15) (end 125.201 123.15) (width 0.5) (layer "B.Cu") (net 3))
 (segment (start 139.2 93.6) (end 139.2 103.7) (width 0.3) (layer "B.Cu") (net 3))
 (segment (start 140.2 141) (end 125.301 141) (width 0.7) (layer "B.Cu") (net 3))
 (segment (start 138.8 103.3) (end 127.1 103.3) (width 0.3) (layer "B.Cu") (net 3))
 (segment (start 125.101 91.601) (end 141.199 91.601) (width 0.3) (layer "B.Cu") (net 3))
 (segment (start 127.65 102.5) (end 127.5 102.35) (width 0.3) (layer "B.Cu") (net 3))
 (segment (start 139.4 140.2) (end 126.1 140.2) (width 0.7) (layer "B.Cu") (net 3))
 (segment (start 127.7 138.6) (end 127.7 130.5) (width 0.7) (layer "B.Cu") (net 3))
 (segment (start 126.9 129.7) (end 139.4 129.7) (width 0.7) (layer "B.Cu") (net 3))
 (segment (start 125.301 141) (end 125.301 128.101) (width 0.7) (layer "B.Cu") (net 3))
 (segment (start 140.8 105.3) (end 125.101 105.3) (width 0.3) (layer "B.Cu") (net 3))
 (segment (start 140.999 128.101) (end 140.999 141.799) (width 0.7) (layer "B.Cu") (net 3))
 (segment (start 139.3 121.95) (end 126.4 121.95) (width 0.5) (layer "B.Cu") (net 3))
 (segment (start 138.6 130.5) (end 138.6 139.4) (width 0.7) (layer "B.Cu") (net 3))
 (segment (start 138.7 112.25) (end 138.7 121.35) (width 0.5) (layer "B.Cu") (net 3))
 (segment (start 139.2 103.7) (end 126.7 103.7) (width 0.3) (layer "B.Cu") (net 3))
 (segment (start 125.5 104.9) (end 125.5 92) (width 0.3) (layer "B.Cu") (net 3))
 (segment (start 141.199 105.699) (end 126.001 105.699) (width 0.3) (layer "B.Cu") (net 3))
 (segment (start 126 141.9) (end 126 144.15) (width 0.7) (layer "B.Cu") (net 3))
 (segment (start 141.199 91.601) (end 141.199 105.699) (width 0.3) (layer "B.Cu") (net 3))
 (segment (start 126.001 105.699) (end 126 105.7) (width 0.3) (layer "B.Cu") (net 3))
 (segment (start 126.4 111.05) (end 139.9 111.05) (width 0.5) (layer "B.Cu") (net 3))
 (segment (start 140 104.5) (end 125.9 104.5) (width 0.3) (layer "B.Cu") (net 3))
 (segment (start 140.4 92.4) (end 140.4 104.9) (width 0.3) (layer "B.Cu") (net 3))
 (segment (start 138.6 139.4) (end 126.9 139.4) (width 0.7) (layer "B.Cu") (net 3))
 (segment (start 141.099 109.851) (end 141.099 123.749) (width 0.5) (layer "B.Cu") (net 3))
 (segment (start 138.7 121.35) (end 127 121.35) (width 0.5) (layer "B.Cu") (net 3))
 (segment (start 140.2 128.9) (end 140.2 141) (width 0.7) (layer "B.Cu") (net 3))
 (segment (start 127.7 130.5) (end 138.6 130.5) (width 0.7) (layer "B.Cu") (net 3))
 (segment (start 137.8 131.3) (end 137.8 138.6) (width 0.7) (layer "B.Cu") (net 3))
 (segment (start 137.8 138.6) (end 127.7 138.6) (width 0.7) (layer "B.Cu") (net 3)))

